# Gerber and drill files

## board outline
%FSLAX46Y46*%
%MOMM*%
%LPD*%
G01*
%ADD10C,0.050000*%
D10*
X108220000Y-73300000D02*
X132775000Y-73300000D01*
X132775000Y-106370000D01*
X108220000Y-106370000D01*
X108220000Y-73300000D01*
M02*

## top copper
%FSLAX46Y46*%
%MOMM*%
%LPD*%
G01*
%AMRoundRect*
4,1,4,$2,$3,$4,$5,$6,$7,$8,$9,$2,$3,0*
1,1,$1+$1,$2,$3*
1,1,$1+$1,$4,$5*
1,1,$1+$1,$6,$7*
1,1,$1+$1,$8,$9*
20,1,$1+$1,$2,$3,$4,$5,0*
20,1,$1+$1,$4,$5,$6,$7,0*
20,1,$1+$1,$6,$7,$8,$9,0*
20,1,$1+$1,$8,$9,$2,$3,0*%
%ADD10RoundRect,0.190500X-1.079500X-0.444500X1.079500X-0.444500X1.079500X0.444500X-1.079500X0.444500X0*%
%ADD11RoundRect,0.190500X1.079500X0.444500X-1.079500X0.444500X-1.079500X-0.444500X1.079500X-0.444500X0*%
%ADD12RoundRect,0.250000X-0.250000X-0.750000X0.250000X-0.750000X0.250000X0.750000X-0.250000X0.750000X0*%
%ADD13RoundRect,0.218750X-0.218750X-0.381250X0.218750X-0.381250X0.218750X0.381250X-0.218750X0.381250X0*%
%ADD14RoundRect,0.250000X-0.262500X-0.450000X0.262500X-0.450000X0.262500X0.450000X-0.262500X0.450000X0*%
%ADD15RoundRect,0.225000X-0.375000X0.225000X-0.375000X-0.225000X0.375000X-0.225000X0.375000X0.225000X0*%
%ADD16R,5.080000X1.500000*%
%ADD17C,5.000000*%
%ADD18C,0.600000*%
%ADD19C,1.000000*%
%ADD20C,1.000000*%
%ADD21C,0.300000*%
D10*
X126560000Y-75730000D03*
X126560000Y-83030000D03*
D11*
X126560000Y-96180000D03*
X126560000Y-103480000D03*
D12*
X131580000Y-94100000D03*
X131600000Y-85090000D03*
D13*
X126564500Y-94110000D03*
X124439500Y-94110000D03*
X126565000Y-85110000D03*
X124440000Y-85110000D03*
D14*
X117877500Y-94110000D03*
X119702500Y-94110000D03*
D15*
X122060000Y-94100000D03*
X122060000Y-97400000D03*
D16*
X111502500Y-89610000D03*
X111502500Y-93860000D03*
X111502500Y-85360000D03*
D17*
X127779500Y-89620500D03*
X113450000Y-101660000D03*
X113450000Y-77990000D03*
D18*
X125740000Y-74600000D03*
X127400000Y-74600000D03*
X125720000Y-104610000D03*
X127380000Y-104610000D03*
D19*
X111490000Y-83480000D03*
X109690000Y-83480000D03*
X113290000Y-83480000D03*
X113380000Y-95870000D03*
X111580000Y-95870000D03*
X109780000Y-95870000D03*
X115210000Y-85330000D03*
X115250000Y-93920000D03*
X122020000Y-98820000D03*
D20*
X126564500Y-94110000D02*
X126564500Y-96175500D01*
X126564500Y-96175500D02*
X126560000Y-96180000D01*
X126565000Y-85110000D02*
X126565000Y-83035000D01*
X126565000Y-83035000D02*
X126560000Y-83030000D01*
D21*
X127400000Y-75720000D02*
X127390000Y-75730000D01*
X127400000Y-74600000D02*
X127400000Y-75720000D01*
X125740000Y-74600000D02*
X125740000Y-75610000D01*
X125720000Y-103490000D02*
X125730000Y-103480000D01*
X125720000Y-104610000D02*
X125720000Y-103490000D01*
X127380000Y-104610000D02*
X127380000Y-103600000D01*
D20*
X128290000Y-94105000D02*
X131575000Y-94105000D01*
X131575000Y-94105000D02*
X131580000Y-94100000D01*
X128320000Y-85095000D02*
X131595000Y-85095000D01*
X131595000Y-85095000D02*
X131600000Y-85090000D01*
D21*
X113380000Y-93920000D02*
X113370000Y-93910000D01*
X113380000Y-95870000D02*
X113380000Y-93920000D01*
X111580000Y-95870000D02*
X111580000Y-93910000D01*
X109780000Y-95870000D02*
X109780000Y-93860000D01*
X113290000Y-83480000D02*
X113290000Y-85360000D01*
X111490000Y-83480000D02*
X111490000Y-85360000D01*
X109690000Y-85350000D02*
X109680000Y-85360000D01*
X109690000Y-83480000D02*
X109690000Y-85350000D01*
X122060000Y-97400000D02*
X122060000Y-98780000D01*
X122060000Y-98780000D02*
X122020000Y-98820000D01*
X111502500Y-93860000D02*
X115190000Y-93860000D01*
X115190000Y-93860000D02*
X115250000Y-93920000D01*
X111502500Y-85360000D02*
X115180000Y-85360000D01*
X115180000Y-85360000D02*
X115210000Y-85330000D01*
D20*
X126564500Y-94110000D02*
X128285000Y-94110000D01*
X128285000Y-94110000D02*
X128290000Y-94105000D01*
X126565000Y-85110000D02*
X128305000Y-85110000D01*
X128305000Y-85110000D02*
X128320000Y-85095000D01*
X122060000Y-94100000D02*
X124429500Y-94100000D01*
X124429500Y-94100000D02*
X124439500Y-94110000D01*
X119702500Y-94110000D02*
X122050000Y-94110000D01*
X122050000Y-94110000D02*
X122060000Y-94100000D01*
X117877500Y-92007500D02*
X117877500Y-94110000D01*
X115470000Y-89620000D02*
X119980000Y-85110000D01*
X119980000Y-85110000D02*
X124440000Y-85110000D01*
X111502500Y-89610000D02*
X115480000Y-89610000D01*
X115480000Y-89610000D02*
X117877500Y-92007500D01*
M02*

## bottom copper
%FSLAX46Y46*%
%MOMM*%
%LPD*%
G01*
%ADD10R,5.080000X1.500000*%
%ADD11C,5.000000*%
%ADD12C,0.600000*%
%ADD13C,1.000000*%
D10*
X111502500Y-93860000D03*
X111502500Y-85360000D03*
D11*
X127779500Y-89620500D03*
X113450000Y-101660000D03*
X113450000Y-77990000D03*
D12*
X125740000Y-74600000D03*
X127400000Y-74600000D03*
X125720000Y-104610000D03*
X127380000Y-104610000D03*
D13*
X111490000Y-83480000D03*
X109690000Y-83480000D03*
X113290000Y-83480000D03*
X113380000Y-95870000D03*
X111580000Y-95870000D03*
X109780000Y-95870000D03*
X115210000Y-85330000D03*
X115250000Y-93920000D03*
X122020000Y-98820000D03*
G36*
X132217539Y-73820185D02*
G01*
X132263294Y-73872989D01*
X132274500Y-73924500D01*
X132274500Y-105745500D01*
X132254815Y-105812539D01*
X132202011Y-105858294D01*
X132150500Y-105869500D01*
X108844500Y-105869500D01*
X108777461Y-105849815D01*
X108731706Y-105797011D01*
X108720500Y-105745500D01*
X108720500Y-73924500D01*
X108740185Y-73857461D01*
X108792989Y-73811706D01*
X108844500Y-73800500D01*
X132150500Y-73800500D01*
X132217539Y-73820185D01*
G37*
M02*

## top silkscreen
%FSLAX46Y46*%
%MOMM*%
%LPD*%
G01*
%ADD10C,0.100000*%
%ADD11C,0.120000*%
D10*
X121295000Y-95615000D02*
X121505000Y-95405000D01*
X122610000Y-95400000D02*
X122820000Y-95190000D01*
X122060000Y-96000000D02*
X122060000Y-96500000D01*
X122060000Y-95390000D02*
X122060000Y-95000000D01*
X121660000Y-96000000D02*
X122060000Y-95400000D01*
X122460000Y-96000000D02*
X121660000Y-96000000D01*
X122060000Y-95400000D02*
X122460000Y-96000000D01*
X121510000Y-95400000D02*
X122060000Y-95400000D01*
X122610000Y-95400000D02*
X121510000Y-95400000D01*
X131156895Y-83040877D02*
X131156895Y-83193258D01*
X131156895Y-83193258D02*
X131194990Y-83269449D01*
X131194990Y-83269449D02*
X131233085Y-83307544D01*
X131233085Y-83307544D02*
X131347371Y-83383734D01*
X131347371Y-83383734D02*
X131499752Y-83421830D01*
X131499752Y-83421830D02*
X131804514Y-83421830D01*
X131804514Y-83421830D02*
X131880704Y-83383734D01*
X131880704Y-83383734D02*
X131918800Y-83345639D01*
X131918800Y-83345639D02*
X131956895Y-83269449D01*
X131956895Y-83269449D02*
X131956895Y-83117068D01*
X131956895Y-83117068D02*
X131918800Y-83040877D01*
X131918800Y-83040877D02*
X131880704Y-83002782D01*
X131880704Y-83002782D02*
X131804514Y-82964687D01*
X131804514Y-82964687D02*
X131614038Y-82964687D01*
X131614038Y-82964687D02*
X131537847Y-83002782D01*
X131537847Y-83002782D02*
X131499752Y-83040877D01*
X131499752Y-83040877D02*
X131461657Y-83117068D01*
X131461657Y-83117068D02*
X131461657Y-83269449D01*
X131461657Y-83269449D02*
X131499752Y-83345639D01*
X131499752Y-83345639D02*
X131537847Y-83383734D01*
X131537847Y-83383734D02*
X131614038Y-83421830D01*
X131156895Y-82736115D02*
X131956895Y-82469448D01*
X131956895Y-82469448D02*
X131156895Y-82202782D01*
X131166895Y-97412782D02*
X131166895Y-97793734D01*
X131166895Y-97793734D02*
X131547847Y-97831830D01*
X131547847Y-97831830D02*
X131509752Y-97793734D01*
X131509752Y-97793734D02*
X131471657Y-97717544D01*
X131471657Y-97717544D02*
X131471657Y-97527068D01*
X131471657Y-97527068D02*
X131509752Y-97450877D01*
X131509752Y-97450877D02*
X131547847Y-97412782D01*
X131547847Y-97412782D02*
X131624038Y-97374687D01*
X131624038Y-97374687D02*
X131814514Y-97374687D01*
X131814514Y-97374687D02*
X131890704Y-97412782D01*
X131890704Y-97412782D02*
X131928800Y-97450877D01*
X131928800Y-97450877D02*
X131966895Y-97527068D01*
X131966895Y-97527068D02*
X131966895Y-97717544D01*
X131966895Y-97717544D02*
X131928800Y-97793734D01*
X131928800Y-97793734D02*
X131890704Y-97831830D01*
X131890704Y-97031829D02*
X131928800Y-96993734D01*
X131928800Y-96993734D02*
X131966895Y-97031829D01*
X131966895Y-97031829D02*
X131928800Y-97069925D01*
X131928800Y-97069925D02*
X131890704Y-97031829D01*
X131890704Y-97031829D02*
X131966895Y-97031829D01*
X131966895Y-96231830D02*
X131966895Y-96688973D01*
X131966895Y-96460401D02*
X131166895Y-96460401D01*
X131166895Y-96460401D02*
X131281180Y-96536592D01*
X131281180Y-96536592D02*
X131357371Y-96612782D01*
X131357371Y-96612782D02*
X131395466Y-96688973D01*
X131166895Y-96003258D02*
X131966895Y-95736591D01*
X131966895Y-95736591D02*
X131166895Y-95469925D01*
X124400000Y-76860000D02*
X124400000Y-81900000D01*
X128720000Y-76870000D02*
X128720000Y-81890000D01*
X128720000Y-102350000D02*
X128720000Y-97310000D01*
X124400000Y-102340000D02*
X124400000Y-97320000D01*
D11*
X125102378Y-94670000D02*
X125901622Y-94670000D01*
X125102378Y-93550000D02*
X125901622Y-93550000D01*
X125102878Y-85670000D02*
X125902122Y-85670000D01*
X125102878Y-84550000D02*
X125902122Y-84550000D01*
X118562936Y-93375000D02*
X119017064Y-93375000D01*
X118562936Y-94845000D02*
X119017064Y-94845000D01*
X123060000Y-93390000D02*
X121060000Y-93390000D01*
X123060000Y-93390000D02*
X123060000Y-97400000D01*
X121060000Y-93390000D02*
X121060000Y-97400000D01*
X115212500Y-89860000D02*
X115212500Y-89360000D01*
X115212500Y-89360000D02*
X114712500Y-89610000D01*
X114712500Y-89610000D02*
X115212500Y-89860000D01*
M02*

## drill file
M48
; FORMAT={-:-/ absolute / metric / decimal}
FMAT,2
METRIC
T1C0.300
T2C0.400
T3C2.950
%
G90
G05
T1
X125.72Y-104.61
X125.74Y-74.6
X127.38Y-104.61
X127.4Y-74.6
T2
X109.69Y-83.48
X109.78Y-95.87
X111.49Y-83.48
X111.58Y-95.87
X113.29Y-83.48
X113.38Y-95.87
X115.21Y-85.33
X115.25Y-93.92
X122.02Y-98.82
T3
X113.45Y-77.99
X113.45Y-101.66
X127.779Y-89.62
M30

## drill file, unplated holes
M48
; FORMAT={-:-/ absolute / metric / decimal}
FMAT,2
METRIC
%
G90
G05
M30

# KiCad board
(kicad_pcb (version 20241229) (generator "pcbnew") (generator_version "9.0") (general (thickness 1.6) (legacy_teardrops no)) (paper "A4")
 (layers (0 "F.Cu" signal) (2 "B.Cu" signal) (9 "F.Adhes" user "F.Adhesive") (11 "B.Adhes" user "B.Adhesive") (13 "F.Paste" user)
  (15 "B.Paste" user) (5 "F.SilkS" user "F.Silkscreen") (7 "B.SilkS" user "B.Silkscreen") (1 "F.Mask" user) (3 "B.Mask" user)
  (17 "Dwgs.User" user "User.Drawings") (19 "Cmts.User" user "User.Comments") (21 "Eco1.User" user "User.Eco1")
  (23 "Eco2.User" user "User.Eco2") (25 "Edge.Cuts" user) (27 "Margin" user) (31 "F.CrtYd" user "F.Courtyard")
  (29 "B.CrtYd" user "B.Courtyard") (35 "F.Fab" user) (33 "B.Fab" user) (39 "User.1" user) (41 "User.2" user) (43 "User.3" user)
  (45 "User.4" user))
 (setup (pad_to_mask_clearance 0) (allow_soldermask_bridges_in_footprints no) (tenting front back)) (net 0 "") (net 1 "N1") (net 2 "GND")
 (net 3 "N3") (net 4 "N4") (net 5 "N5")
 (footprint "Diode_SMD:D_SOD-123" (layer "F.Cu") (at 122.06 95.75 -90)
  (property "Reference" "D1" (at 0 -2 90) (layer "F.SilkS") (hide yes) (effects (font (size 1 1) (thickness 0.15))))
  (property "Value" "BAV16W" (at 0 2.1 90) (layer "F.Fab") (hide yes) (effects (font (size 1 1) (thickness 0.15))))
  (fp_line (start -2.36 1) (end 1.65 1) (stroke (width 0.12) (type solid)) (layer "F.SilkS"))
  (fp_line (start -2.36 -1) (end -2.36 1) (stroke (width 0.12) (type solid)) (layer "F.SilkS"))
  (fp_line (start -2.36 -1) (end 1.65 -1) (stroke (width 0.12) (type solid)) (layer "F.SilkS"))
  (pad "1" smd roundrect (at -1.65 0 270) (size 0.9 1.2) (layers "F.Cu" "F.Mask" "F.Paste") (roundrect_rratio 0.25) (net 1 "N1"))
  (pad "2" smd roundrect (at 1.65 0 270) (size 0.9 1.2) (layers "F.Cu" "F.Mask" "F.Paste") (roundrect_rratio 0.25) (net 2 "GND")))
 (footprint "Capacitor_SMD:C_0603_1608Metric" (layer "F.Cu") (at 126.56 79.38 -90)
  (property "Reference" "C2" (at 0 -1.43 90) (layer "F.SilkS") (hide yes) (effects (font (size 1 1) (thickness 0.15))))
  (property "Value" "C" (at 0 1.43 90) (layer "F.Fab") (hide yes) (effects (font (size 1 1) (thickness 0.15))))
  (fp_line (start -2.52 2.16) (end 2.52 2.16) (stroke (width 0.1) (type solid)) (layer "F.SilkS"))
  (fp_line (start -2.51 -2.16) (end 2.51 -2.16) (stroke (width 0.1) (type solid)) (layer "F.SilkS"))
  (pad "1" smd roundrect (at 3.65 0) (size 2.54 1.27) (layers "F.Cu" "F.Mask" "F.Paste") (roundrect_rratio 0.15) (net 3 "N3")
   (thermal_bridge_angle 45))
  (pad "2" smd roundrect (at -3.65 0) (size 2.54 1.27) (layers "F.Cu" "F.Mask" "F.Paste") (roundrect_rratio 0.15) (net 2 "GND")
   (thermal_bridge_angle 45)))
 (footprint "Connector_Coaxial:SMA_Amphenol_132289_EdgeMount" (layer "F.Cu") (at 111.5025 89.61 180)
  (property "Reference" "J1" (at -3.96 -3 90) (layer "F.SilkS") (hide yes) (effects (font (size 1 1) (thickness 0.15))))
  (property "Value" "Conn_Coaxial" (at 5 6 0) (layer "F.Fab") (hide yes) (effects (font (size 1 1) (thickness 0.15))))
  (fp_line (start -3.21 0) (end -3.71 -0.25) (stroke (width 0.12) (type solid)) (layer "F.SilkS"))
  (fp_line (start -3.71 0.25) (end -3.21 0) (stroke (width 0.12) (type solid)) (layer "F.SilkS"))
  (fp_line (start -3.71 -0.25) (end -3.71 0.25) (stroke (width 0.12) (type solid)) (layer "F.SilkS"))
  (pad "1" smd rect (at 0 0 270) (size 1.5 5.08) (layers "F.Cu" "F.Mask" "F.Paste") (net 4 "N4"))
  (pad "2" smd rect (at 0 -4.25 270) (size 1.5 5.08) (layers "F.Cu" "F.Mask" "F.Paste") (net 2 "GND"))
  (pad "2" smd rect (at 0 -4.25 270) (size 1.5 5.08) (layers "B.Cu" "B.Mask" "B.Paste") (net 2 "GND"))
  (pad "2" smd rect (at 0 4.25 270) (size 1.5 5.08) (layers "F.Cu" "F.Mask" "F.Paste") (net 2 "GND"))
  (pad "2" smd rect (at 0 4.25 270) (size 1.5 5.08) (layers "B.Cu" "B.Mask" "B.Paste") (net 2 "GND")))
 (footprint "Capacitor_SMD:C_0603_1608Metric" (layer "F.Cu") (at 126.56 99.83 90)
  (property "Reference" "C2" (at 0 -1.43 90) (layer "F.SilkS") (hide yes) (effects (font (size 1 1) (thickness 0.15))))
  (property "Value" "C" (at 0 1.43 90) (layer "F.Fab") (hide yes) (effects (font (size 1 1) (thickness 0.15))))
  (fp_line (start -2.51 -2.16) (end 2.51 -2.16) (stroke (width 0.1) (type solid)) (layer "F.SilkS"))
  (fp_line (start -2.52 2.16) (end 2.52 2.16) (stroke (width 0.1) (type solid)) (layer "F.SilkS"))
  (pad "1" smd roundrect (at 3.65 0 180) (size 2.54 1.27) (layers "F.Cu" "F.Mask" "F.Paste") (roundrect_rratio 0.15) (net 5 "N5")
   (thermal_bridge_angle 45))
  (pad "2" smd roundrect (at -3.65 0 180) (size 2.54 1.27) (layers "F.Cu" "F.Mask" "F.Paste") (roundrect_rratio 0.15) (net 2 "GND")
   (thermal_bridge_angle 45)))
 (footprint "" (layer "F.Cu") (at 130.72 94.1)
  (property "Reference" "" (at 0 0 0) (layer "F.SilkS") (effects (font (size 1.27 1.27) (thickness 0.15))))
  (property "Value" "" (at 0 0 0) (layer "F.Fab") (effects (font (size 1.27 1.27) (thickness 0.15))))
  (pad "2" smd roundrect (at 0 0) (size 2.72 1.92) (layers "F.Cu" "F.Mask" "F.Paste") (roundrect_rratio 0.25) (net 5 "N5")))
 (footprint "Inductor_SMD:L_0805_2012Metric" (layer "F.Cu") (at 125.5025 85.11)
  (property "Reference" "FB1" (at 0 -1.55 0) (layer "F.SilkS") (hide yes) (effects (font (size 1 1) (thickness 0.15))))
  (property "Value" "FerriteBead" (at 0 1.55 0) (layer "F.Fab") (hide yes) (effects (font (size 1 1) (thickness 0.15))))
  (fp_line (start -0.399622 -0.56) (end 0.399622 -0.56) (stroke (width 0.12) (type solid)) (layer "F.SilkS"))
  (fp_line (start -0.399622 0.56) (end 0.399622 0.56) (stroke (width 0.12) (type solid)) (layer "F.SilkS"))
  (pad "1" smd roundrect (at -1.0625 0) (size 0.875 1.2) (layers "F.Cu" "F.Mask" "F.Paste") (roundrect_rratio 0.25) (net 4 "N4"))
  (pad "2" smd roundrect (at 1.0625 0) (size 0.875 1.2) (layers "F.Cu" "F.Mask" "F.Paste") (roundrect_rratio 0.25) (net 3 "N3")))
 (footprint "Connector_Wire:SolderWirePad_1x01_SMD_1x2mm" (layer "F.Cu") (at 131.6 85.09)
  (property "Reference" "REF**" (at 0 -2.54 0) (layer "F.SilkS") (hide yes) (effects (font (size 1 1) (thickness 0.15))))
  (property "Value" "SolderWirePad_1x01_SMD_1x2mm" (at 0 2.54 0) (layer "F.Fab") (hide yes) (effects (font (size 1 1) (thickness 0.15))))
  (pad "1" smd roundrect (at -0.86 -0.04) (size 2.72 1.92) (layers "F.Cu" "F.Mask" "F.Paste") (roundrect_rratio 0.25) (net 3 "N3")))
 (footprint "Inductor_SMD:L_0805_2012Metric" (layer "F.Cu") (at 125.502 94.11)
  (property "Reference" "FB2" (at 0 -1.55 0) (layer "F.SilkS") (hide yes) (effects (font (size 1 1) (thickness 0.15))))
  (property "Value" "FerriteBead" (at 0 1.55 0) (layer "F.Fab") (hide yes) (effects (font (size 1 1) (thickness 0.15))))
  (fp_line (start -0.399622 -0.56) (end 0.399622 -0.56) (stroke (width 0.12) (type solid)) (layer "F.SilkS"))
  (fp_line (start -0.399622 0.56) (end 0.399622 0.56) (stroke (width 0.12) (type solid)) (layer "F.SilkS"))
  (pad "1" smd roundrect (at -1.0625 0) (size 0.875 1.2) (layers "F.Cu" "F.Mask" "F.Paste") (roundrect_rratio 0.25) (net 1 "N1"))
  (pad "2" smd roundrect (at 1.0625 0) (size 0.875 1.2) (layers "F.Cu" "F.Mask" "F.Paste") (roundrect_rratio 0.25) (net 5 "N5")))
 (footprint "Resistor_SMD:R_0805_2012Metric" (layer "F.Cu") (at 118.79 94.11)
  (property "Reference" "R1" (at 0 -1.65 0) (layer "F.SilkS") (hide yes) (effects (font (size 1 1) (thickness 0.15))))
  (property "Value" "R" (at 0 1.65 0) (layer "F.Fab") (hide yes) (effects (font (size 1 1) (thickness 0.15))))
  (fp_line (start -0.227064 -0.735) (end 0.227064 -0.735) (stroke (width 0.12) (type solid)) (layer "F.SilkS"))
  (fp_line (start -0.227064 0.735) (end 0.227064 0.735) (stroke (width 0.12) (type solid)) (layer "F.SilkS"))
  (pad "1" smd roundrect (at -0.9125 0) (size 1.025 1.4) (layers "F.Cu" "F.Mask" "F.Paste") (roundrect_rratio 0.243902) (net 4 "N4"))
  (pad "2" smd roundrect (at 0.9125 0) (size 1.025 1.4) (layers "F.Cu" "F.Mask" "F.Paste") (roundrect_rratio 0.243902) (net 1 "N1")))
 (gr_line (start 122.06 96) (end 122.06 96.5) (stroke (width 0.1) (type default)) (layer "F.SilkS"))
 (gr_line (start 121.51 95.4) (end 122.06 95.4) (stroke (width 0.1) (type default)) (layer "F.SilkS"))
 (gr_line (start 122.61 95.4) (end 121.51 95.4) (stroke (width 0.1) (type default)) (layer "F.SilkS"))
 (gr_line (start 122.46 96) (end 121.66 96) (stroke (width 0.1) (type default)) (layer "F.SilkS"))
 (gr_line (start 122.06 95.39) (end 122.06 95) (stroke (width 0.1) (type default)) (layer "F.SilkS"))
 (gr_line (start 121.66 96) (end 122.06 95.4) (stroke (width 0.1) (type default)) (layer "F.SilkS"))
 (gr_line (start 121.295 95.615) (end 121.505 95.405) (stroke (width 0.1) (type default)) (layer "F.SilkS"))
 (gr_line (start 122.06 95.4) (end 122.46 96) (stroke (width 0.1) (type default)) (layer "F.SilkS"))
 (gr_line (start 122.61 95.4) (end 122.82 95.19) (stroke (width 0.1) (type default)) (layer "F.SilkS"))
 (gr_rect (start 108.22 73.3) (end 132.775 106.37) (stroke (width 0.05) (type default)) (fill no) (layer "Edge.Cuts"))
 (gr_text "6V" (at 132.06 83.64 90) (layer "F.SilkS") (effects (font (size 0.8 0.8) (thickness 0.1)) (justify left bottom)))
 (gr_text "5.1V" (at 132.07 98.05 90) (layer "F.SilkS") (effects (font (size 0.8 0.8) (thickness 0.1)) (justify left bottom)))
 (segment (start 111.58 95.87) (end 111.58 93.91) (width 0.3) (layer "F.Cu") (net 2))
 (segment (start 111.49 83.48) (end 111.49 85.36) (width 0.3) (layer "F.Cu") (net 2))
 (segment (start 122.06 98.78) (end 122.02 98.82) (width 0.3) (layer "F.Cu") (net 2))
 (segment (start 111.5025 85.36) (end 115.18 85.36) (width 0.3) (layer "F.Cu") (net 2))
 (segment (start 125.72 104.61) (end 125.72 103.49) (width 0.3) (layer "F.Cu") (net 2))
 (segment (start 115.19 93.86) (end 115.25 93.92) (width 0.3) (layer "F.Cu") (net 2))
 (segment (start 122.06 97.4) (end 122.06 98.78) (width 0.3) (layer "F.Cu") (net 2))
 (segment (start 125.72 103.49) (end 125.73 103.48) (width 0.3) (layer "F.Cu") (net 2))
 (segment (start 113.29 83.48) (end 113.29 85.36) (width 0.3) (layer "F.Cu") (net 2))
 (segment (start 109.78 95.87) (end 109.78 93.86) (width 0.3) (layer "F.Cu") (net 2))
 (segment (start 115.18 85.36) (end 115.21 85.33) (width 0.3) (layer "F.Cu") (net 2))
 (segment (start 111.5025 93.86) (end 115.19 93.86) (width 0.3) (layer "F.Cu") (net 2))
 (segment (start 109.69 83.48) (end 109.69 85.35) (width 0.3) (layer "F.Cu") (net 2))
 (segment (start 127.38 104.61) (end 127.38 103.6) (width 0.3) (layer "F.Cu") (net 2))
 (segment (start 113.38 93.92) (end 113.37 93.91) (width 0.3) (layer "F.Cu") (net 2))
 (segment (start 127.4 74.6) (end 127.4 75.72) (width 0.3) (layer "F.Cu") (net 2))
 (segment (start 109.69 85.35) (end 109.68 85.36) (width 0.3) (layer "F.Cu") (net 2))
 (segment (start 127.4 75.72) (end 127.39 75.73) (width 0.3) (layer "F.Cu") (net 2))
 (segment (start 125.74 74.6) (end 125.74 75.61) (width 0.3) (layer "F.Cu") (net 2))
 (segment (start 113.38 95.87) (end 113.38 93.92) (width 0.3) (layer "F.Cu") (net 2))
 (via (at 113.45 77.99) (size 5) (drill 2.95) (layers "F.Cu" "B.Cu") (free yes) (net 2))
 (via (at 115.21 85.33) (size 1) (drill 0.4) (layers "F.Cu" "B.Cu") (free yes) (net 2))
 (via (at 113.38 95.87) (size 1) (drill 0.4) (layers "F.Cu" "B.Cu") (free yes) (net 2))
 (via (at 109.78 95.87) (size 1) (drill 0.4) (layers "F.Cu" "B.Cu") (free yes) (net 2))
 (via (at 115.25 93.92) (size 1) (drill 0.4) (layers "F.Cu" "B.Cu") (free yes) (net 2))
 (via (at 127.38 104.61) (size 0.6) (drill 0.3) (layers "F.Cu" "B.Cu") (free yes) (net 2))
 (via (at 127.4 74.6) (size 0.6) (drill 0.3) (layers "F.Cu" "B.Cu") (free yes) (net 2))
 (via (at 122.02 98.82) (size 1) (drill 0.4) (layers "F.Cu" "B.Cu") (free yes) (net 2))
 (via (at 125.72 104.61) (size 0.6) (drill 0.3) (layers "F.Cu" "B.Cu") (free yes) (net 2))
 (via (at 109.69 83.48) (size 1) (drill 0.4) (layers "F.Cu" "B.Cu") (free yes) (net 2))
 (via (at 113.45 101.66) (size 5) (drill 2.95) (layers "F.Cu" "B.Cu") (free yes) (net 2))
 (via (at 111.49 83.48) (size 1) (drill 0.4) (layers "F.Cu" "B.Cu") (free yes) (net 2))
 (via (at 111.58 95.87) (size 1) (drill 0.4) (layers "F.Cu" "B.Cu") (free yes) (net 2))
 (via (at 113.29 83.48) (size 1) (drill 0.4) (layers "F.Cu" "B.Cu") (free yes) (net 2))
 (via (at 127.7795 89.6205) (size 5) (drill 2.95) (layers "F.Cu" "B.Cu") (free yes) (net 2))
 (via (at 125.74 74.6) (size 0.6) (drill 0.3) (layers "F.Cu" "B.Cu") (free yes) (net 2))
 (segment (start 126.565 85.11) (end 126.565 83.035) (width 1) (layer "F.Cu") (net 3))
 (segment (start 128.305 85.11) (end 128.32 85.095) (width 1) (layer "F.Cu") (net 3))
 (segment (start 128.32 85.095) (end 131.595 85.095) (width 1) (layer "F.Cu") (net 3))
 (segment (start 126.565 85.11) (end 128.305 85.11) (width 1) (layer "F.Cu") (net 3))
 (segment (start 126.565 83.035) (end 126.56 83.03) (width 1) (layer "F.Cu") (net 3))
 (segment (start 128.29 94.105) (end 131.575 94.105) (width 1) (layer "F.Cu") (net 5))
 (segment (start 126.5645 94.11) (end 128.285 94.11) (width 1) (layer "F.Cu") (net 5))
 (segment (start 126.5645 94.11) (end 126.5645 96.1755) (width 1) (layer "F.Cu") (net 5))
 (segment (start 131.575 94.105) (end 131.58 94.1) (width 1) (layer "F.Cu") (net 5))
 (segment (start 126.5645 96.1755) (end 126.56 96.18) (width 1) (layer "F.Cu") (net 5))
 (segment (start 128.285 94.11) (end 128.29 94.105) (width 1) (layer "F.Cu") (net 5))
 (segment (start 124.4295 94.1) (end 124.4395 94.11) (width 1) (layer "F.Cu") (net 1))
 (segment (start 119.7025 94.11) (end 122.05 94.11) (width 1) (layer "F.Cu") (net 1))
 (segment (start 122.05 94.11) (end 122.06 94.1) (width 1) (layer "F.Cu") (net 1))
 (segment (start 122.06 94.1) (end 124.4295 94.1) (width 1) (layer "F.Cu") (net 1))
 (segment (start 119.98 85.11) (end 124.44 85.11) (width 1) (layer "F.Cu") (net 4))
 (segment (start 115.47 89.62) (end 119.98 85.11) (width 1) (layer "F.Cu") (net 4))
 (segment (start 117.8775 92.0075) (end 117.8775 94.11) (width 1) (layer "F.Cu") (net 4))
 (segment (start 115.48 89.61) (end 117.8775 92.0075) (width 1) (layer "F.Cu") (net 4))
 (segment (start 111.5025 89.61) (end 115.48 89.61) (width 1) (layer "F.Cu") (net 4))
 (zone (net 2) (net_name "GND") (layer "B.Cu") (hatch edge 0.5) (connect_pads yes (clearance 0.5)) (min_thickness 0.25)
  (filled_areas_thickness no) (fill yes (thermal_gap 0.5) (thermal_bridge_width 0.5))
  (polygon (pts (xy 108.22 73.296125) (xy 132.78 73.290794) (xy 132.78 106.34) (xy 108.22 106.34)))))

